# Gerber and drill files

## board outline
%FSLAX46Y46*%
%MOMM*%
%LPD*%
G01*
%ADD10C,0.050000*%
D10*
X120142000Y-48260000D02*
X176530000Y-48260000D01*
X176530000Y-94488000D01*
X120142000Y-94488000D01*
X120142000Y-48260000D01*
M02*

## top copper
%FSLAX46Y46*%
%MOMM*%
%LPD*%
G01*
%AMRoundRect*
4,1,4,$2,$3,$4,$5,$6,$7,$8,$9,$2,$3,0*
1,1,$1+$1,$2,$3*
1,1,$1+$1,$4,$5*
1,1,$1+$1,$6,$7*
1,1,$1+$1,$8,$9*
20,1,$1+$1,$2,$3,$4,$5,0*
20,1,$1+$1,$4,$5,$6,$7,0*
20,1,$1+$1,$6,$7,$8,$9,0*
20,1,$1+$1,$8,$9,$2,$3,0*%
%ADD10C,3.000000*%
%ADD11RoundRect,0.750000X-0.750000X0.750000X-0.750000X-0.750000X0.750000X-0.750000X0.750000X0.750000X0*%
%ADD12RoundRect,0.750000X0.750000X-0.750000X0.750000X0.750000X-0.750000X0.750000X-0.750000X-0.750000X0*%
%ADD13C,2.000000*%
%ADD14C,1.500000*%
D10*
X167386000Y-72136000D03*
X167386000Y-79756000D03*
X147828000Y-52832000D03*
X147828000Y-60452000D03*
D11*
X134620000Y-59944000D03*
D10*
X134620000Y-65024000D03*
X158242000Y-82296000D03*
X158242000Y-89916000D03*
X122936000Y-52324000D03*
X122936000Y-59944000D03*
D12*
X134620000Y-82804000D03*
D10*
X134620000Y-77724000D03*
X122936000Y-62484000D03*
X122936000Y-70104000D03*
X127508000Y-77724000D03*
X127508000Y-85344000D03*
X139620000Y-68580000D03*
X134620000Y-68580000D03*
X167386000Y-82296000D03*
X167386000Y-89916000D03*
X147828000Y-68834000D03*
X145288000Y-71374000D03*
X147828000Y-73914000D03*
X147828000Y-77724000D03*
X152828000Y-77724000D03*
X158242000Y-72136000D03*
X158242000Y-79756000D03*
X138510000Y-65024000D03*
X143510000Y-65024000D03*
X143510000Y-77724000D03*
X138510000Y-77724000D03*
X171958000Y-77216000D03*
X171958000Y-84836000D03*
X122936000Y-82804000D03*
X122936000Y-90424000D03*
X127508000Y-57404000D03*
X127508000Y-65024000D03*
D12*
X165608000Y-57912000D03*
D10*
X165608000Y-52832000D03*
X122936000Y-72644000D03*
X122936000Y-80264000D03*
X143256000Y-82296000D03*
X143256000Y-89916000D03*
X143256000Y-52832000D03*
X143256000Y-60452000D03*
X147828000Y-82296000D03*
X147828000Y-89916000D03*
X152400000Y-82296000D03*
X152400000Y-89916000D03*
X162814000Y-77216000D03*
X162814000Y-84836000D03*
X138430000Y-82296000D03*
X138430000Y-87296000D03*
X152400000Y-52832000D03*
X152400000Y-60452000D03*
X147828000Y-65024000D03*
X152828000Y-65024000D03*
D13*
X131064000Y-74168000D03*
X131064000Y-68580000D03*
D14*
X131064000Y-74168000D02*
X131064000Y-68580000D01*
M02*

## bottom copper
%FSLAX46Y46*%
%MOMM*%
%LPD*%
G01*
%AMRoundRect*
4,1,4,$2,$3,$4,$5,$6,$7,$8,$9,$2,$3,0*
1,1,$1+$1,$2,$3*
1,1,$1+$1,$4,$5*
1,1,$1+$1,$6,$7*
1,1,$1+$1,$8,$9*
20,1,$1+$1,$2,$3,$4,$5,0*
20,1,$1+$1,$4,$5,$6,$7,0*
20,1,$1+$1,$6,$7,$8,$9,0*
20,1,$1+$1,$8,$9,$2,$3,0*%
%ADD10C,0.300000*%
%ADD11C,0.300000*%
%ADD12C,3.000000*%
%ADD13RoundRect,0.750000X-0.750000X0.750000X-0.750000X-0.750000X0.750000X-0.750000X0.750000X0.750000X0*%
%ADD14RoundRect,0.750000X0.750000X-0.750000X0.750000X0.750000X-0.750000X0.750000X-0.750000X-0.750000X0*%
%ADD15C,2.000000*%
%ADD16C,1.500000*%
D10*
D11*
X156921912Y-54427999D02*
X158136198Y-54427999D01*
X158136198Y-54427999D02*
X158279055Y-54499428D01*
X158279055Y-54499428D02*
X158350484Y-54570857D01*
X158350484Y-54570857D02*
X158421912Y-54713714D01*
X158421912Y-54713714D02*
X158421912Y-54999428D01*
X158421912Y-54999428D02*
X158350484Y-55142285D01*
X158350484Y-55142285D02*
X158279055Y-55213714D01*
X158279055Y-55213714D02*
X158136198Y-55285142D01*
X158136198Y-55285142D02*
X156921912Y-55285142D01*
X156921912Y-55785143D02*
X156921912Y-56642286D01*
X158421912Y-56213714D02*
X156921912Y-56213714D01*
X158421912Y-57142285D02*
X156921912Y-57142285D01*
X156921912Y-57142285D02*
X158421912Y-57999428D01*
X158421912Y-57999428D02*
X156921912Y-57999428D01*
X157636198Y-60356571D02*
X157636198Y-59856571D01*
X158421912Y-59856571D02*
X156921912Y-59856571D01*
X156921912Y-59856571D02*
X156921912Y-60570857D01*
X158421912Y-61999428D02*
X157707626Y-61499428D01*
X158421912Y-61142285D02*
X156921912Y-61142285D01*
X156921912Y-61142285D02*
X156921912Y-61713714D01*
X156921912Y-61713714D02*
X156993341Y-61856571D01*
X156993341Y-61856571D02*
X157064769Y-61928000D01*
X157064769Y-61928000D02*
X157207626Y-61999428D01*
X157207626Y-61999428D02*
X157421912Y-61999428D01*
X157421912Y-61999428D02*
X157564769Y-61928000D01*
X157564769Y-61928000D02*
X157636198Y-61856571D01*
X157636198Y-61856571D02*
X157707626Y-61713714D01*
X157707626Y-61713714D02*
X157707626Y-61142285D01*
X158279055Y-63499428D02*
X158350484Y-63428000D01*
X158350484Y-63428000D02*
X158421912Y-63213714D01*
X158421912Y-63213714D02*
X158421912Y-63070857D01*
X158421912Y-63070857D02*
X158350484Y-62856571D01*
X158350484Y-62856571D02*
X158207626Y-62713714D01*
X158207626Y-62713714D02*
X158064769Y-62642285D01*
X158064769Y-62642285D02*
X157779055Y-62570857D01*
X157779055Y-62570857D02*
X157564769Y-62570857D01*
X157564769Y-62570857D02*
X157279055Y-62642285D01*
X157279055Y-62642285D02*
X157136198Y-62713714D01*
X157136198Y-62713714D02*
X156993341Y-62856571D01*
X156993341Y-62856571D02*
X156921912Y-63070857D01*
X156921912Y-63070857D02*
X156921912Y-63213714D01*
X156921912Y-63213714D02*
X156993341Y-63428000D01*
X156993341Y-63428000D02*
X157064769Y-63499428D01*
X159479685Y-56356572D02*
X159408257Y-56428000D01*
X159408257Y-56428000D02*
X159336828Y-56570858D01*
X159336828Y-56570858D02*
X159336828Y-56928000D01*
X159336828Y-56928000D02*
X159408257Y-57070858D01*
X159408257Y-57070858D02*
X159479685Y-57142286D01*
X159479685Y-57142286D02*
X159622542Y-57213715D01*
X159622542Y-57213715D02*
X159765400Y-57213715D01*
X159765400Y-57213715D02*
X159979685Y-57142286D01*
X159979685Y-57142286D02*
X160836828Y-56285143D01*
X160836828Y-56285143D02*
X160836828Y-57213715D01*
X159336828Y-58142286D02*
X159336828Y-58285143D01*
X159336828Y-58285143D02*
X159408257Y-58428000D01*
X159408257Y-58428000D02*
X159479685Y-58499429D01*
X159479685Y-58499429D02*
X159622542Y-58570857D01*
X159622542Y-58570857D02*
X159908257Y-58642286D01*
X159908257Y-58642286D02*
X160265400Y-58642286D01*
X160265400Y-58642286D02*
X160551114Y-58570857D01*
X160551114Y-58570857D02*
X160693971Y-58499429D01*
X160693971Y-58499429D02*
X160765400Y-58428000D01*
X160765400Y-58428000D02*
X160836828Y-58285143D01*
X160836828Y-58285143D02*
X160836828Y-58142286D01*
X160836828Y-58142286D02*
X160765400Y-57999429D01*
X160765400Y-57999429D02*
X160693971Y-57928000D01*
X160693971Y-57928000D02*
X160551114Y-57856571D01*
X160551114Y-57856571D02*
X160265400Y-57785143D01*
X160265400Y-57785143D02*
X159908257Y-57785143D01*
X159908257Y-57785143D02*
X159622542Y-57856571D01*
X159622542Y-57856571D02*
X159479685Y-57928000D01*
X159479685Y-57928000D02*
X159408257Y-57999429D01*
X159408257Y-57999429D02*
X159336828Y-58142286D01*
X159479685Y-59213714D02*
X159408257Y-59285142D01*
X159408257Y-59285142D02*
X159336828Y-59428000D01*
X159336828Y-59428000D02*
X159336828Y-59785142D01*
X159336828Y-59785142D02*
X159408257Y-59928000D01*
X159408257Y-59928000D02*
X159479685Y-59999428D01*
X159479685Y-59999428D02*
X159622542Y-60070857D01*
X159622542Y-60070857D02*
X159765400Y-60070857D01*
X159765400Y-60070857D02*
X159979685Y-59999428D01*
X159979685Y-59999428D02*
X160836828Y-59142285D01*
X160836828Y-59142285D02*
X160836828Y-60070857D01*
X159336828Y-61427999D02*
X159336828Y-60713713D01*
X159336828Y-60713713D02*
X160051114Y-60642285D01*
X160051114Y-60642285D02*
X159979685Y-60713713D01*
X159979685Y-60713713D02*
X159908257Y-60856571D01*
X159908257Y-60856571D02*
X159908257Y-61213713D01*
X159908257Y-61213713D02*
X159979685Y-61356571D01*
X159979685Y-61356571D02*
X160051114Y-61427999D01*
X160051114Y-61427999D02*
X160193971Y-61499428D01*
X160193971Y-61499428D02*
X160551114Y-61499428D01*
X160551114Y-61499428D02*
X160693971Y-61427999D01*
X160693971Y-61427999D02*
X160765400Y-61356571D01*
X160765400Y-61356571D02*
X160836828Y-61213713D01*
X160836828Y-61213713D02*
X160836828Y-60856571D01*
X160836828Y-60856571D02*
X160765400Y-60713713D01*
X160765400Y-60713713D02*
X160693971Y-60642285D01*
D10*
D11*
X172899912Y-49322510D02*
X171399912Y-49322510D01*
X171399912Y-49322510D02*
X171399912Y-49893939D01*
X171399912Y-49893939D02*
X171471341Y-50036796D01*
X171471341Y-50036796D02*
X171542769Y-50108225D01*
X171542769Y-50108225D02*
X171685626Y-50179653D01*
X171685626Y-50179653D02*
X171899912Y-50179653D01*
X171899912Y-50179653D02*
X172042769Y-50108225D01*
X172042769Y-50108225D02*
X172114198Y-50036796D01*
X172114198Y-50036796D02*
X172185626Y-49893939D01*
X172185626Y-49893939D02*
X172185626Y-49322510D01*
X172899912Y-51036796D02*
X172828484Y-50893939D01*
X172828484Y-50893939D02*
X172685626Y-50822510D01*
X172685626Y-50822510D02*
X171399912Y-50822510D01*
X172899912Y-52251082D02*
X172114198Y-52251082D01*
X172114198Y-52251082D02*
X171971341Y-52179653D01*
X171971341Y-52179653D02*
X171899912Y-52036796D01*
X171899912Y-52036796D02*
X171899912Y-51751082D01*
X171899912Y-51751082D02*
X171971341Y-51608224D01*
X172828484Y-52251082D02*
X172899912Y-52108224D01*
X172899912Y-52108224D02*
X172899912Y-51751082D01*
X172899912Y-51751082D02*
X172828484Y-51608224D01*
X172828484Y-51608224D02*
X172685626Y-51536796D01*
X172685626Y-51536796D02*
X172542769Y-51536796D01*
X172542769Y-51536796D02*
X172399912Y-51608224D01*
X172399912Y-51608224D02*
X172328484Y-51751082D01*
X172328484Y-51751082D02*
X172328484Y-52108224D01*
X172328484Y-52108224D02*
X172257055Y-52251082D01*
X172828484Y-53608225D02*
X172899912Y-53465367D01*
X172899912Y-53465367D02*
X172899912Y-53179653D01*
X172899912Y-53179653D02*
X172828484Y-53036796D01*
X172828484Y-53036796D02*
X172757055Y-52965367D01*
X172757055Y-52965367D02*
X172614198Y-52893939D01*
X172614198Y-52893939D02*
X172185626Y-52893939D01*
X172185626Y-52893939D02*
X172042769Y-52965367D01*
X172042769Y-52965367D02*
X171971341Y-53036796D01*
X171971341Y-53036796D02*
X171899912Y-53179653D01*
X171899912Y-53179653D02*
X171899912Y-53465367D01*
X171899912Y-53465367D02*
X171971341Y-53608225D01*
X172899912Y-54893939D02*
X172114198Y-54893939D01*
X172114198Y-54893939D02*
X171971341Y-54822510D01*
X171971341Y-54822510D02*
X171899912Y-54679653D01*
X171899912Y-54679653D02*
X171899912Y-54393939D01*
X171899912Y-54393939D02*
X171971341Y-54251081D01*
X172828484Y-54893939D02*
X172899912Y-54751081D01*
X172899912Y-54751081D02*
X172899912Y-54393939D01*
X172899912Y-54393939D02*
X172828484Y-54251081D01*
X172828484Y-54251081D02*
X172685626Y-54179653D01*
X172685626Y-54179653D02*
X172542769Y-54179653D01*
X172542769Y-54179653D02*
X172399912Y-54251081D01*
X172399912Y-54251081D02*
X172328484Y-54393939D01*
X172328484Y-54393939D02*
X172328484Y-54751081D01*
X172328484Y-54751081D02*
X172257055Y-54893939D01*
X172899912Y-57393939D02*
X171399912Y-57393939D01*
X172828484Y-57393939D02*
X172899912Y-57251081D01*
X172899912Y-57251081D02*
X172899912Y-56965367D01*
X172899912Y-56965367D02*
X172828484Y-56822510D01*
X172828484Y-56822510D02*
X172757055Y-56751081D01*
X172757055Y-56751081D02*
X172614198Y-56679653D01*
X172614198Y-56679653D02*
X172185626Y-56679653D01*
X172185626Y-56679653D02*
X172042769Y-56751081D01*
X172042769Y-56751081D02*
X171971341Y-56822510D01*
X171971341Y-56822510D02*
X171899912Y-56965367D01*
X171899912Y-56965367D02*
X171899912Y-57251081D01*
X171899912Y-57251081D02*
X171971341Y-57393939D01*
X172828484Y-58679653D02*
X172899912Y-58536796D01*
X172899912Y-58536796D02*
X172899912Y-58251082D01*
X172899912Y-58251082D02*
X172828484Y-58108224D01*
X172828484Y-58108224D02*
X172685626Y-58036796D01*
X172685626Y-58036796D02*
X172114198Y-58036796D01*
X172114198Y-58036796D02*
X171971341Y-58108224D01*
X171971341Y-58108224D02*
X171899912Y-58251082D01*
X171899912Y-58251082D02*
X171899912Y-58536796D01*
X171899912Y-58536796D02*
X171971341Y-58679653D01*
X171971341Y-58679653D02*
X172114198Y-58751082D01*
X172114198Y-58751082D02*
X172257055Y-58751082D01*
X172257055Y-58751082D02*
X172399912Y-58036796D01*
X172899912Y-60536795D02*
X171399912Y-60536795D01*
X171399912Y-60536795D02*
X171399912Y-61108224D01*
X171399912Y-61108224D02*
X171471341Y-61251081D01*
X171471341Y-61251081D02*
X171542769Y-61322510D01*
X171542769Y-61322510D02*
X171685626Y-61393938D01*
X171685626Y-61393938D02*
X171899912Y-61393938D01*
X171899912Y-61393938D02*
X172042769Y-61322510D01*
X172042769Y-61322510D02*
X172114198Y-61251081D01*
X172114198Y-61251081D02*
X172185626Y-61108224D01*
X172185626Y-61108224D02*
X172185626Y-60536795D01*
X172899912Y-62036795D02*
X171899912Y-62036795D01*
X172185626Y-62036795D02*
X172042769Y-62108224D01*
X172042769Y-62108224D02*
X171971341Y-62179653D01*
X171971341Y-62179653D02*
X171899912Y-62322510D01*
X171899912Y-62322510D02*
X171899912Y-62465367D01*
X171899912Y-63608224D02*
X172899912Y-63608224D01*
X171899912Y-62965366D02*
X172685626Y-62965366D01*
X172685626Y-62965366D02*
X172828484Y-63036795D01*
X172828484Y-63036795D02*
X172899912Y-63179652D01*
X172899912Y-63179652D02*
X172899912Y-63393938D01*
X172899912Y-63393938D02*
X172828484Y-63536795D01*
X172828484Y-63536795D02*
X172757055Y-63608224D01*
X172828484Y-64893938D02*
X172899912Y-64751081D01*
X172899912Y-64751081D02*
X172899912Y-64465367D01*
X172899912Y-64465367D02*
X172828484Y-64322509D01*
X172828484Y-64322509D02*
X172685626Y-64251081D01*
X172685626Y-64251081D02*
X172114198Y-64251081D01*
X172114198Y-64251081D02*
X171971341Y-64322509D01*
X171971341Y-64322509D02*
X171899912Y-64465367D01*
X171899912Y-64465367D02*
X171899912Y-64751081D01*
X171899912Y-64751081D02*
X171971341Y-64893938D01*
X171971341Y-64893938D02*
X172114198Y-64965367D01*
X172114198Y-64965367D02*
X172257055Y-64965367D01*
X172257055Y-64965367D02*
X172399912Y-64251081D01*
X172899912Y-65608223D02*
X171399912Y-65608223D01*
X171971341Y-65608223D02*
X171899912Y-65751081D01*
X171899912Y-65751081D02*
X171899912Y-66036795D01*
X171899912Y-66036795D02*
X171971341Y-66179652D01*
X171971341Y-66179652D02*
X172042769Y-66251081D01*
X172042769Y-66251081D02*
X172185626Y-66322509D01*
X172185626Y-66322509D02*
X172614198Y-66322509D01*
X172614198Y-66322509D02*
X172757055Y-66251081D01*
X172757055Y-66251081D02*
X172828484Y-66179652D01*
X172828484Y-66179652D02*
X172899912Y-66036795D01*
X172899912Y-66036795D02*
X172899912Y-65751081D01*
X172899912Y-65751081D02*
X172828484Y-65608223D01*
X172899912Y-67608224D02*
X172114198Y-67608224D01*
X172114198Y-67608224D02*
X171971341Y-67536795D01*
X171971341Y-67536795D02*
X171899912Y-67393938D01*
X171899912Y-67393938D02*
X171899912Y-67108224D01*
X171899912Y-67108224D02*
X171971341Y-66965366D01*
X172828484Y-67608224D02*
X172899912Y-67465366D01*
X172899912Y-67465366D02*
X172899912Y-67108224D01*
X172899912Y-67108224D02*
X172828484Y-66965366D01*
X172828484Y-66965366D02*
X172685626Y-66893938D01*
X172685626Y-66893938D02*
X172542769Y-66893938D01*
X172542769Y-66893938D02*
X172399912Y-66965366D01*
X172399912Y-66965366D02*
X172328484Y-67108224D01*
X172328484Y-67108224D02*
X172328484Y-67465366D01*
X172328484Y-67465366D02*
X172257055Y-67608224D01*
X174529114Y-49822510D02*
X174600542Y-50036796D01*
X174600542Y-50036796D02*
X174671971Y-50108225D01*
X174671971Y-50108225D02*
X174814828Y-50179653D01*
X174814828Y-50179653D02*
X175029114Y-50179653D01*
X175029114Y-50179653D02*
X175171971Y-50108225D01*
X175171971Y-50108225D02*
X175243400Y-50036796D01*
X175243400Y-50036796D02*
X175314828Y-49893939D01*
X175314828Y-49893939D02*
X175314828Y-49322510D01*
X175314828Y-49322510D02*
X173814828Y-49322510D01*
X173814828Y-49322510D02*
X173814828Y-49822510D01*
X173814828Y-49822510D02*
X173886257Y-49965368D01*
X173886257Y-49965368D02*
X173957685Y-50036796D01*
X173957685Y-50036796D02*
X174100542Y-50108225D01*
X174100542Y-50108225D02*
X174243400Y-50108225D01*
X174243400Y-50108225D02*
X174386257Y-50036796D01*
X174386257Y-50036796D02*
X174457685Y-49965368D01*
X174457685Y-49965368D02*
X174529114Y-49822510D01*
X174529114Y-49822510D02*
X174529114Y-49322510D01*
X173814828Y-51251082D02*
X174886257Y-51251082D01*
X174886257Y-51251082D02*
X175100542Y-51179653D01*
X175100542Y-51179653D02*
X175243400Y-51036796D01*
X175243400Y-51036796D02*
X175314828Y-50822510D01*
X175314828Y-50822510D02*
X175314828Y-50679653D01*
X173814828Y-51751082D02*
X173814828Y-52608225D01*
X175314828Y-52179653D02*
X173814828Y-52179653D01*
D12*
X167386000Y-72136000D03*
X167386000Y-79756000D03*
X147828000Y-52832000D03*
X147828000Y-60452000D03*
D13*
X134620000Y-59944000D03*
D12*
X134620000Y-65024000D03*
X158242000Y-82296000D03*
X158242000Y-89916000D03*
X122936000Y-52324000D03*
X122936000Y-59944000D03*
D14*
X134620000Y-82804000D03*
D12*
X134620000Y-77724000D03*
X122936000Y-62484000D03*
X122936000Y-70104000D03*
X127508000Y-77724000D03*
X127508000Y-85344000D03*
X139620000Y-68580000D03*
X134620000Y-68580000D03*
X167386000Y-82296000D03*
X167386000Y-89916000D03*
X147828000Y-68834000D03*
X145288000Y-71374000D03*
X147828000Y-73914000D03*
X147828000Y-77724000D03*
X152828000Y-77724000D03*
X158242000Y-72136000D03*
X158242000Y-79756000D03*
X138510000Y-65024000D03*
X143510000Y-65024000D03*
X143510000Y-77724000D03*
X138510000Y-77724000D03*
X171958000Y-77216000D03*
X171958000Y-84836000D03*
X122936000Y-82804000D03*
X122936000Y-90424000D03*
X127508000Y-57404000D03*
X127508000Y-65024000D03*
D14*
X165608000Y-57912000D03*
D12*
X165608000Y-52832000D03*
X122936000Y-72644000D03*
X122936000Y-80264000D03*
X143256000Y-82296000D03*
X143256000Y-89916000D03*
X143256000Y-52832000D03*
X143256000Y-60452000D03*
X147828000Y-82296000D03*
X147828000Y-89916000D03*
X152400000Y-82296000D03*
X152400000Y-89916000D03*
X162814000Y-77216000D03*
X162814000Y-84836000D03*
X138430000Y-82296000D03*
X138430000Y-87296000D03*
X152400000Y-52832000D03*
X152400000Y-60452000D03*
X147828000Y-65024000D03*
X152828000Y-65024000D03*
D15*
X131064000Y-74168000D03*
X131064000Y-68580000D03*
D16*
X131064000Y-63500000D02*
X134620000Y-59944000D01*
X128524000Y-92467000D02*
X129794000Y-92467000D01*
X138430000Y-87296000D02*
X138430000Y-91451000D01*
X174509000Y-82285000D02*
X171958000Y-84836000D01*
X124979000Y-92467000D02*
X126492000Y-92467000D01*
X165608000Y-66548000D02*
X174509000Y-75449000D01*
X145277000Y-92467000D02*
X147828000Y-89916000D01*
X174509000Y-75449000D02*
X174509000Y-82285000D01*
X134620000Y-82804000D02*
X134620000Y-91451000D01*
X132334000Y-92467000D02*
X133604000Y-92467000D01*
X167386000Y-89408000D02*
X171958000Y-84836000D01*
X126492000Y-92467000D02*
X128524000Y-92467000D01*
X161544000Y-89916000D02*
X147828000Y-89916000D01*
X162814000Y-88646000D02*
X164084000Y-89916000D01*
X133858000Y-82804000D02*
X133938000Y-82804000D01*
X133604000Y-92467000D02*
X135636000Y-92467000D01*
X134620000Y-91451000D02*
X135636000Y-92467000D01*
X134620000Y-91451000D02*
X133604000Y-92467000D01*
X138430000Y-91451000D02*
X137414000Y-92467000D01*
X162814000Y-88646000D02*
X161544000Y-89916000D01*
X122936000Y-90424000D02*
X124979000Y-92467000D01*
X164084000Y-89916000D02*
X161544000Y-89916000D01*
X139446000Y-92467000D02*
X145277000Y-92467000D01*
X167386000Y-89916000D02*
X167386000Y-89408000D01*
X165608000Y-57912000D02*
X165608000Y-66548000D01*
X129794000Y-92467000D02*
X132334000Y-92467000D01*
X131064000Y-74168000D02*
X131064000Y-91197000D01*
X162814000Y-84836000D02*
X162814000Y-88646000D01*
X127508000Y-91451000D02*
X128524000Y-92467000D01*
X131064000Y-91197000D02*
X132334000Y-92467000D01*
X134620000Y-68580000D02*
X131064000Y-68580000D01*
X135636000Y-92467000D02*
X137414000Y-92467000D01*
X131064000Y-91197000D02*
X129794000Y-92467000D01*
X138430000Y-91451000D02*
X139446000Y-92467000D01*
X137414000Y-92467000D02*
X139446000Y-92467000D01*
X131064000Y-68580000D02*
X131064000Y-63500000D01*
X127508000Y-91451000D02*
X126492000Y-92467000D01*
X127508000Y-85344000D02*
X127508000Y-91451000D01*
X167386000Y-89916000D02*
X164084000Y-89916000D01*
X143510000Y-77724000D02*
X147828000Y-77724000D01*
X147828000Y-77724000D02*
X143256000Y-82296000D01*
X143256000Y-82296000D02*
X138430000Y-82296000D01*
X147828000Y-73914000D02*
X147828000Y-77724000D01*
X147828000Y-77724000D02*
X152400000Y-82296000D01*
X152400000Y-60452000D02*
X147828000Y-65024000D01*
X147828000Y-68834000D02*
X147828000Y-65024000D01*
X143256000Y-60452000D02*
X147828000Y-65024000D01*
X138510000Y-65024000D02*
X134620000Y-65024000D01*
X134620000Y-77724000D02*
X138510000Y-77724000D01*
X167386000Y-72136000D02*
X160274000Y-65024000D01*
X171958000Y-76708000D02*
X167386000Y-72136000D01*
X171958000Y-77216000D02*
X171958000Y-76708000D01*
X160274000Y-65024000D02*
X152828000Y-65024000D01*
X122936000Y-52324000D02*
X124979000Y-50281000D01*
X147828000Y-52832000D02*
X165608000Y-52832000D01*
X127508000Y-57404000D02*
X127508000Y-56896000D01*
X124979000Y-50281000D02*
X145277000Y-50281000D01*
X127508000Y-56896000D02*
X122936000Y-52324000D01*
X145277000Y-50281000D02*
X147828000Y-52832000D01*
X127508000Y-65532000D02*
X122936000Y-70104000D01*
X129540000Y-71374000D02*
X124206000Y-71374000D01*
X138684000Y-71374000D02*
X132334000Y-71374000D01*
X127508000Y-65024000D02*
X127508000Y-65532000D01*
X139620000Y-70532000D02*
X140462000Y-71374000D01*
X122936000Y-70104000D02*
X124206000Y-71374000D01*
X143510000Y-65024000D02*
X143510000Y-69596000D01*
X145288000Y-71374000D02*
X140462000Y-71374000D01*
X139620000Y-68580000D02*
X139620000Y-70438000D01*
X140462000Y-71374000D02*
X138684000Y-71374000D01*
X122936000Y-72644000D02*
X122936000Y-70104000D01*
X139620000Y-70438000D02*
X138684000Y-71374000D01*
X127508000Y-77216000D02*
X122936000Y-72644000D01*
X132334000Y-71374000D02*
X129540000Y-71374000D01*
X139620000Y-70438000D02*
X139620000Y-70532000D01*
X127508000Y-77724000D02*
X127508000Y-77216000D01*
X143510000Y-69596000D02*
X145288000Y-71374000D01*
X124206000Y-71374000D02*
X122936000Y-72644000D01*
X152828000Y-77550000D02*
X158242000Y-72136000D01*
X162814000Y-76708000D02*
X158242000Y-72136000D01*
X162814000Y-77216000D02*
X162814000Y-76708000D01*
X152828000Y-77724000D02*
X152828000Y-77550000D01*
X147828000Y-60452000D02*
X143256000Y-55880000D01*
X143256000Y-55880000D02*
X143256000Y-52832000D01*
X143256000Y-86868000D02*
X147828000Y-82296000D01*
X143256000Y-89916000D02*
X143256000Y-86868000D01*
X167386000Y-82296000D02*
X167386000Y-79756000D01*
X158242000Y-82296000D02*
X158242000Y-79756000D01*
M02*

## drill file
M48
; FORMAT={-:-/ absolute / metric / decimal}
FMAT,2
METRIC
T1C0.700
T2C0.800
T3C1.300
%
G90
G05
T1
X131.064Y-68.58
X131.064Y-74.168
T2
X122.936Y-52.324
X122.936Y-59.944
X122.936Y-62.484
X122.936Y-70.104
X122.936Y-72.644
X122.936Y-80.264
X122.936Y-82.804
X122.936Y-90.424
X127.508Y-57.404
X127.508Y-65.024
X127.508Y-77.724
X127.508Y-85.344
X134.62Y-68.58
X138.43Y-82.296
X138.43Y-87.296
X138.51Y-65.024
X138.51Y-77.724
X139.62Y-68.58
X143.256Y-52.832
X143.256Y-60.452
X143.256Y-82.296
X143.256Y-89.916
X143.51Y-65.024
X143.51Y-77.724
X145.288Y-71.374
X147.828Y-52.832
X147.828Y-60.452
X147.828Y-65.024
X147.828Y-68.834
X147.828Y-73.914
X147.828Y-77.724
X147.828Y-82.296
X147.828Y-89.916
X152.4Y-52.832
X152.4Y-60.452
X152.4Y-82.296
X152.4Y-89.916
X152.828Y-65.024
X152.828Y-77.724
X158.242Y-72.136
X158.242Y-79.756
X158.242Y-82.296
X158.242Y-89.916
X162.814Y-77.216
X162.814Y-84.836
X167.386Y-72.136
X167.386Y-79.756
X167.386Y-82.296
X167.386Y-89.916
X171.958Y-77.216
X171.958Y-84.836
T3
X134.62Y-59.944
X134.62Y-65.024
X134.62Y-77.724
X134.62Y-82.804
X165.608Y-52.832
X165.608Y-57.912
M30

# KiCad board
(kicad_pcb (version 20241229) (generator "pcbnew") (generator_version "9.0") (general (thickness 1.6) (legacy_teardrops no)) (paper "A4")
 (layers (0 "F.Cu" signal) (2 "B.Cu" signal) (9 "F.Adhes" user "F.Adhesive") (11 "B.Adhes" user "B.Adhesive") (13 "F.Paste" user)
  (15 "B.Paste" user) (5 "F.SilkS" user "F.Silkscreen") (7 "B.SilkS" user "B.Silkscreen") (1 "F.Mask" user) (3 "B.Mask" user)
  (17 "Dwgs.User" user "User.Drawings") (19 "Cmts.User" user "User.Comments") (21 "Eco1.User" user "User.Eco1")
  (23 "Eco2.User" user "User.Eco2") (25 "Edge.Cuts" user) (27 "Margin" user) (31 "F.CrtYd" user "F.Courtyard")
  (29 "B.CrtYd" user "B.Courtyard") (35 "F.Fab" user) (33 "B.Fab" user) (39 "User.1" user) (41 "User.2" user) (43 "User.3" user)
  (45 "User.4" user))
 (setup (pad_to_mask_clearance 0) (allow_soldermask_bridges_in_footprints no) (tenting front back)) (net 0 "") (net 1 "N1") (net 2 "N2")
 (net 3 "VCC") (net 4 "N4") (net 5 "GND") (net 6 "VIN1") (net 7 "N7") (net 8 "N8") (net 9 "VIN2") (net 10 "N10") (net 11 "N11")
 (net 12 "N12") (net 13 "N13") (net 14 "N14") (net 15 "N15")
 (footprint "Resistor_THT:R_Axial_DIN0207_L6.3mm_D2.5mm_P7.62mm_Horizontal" (layer "F.Cu") (at 167.386 72.136 -90)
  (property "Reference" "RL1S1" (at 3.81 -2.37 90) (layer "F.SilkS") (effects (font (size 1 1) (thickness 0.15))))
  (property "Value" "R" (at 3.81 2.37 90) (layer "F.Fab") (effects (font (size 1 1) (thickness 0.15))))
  (pad "1" thru_hole circle (at 0 0 270) (size 3 3) (drill 0.8) (layers "*.Cu" "*.Mask") (remove_unused_layers no) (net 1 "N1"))
  (pad "2" thru_hole circle (at 7.62 0 270) (size 3 3) (drill 0.8) (layers "*.Cu" "*.Mask") (remove_unused_layers no) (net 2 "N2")))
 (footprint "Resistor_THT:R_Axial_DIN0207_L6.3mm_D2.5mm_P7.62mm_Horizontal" (layer "F.Cu") (at 147.828 52.832 -90)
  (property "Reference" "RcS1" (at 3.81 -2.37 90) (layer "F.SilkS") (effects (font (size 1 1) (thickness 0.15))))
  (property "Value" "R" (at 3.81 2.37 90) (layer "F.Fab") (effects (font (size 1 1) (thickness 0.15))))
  (pad "1" thru_hole circle (at 0 0 270) (size 3 3) (drill 0.8) (layers "*.Cu" "*.Mask") (remove_unused_layers no) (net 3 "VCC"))
  (pad "2" thru_hole circle (at 7.62 0 270) (size 3 3) (drill 0.8) (layers "*.Cu" "*.Mask") (remove_unused_layers no) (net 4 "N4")))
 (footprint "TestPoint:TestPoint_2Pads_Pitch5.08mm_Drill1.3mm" (layer "F.Cu") (at 134.62 59.944 -90)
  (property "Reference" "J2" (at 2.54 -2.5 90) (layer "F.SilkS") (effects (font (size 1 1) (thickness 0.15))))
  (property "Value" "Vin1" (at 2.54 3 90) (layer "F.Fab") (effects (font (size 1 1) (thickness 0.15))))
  (pad "1" thru_hole roundrect (at 0 0 270) (size 3 3) (drill 1.3) (layers "*.Cu" "*.Mask") (remove_unused_layers no)
   (roundrect_rratio 0.25) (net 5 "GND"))
  (pad "2" thru_hole circle (at 5.08 0 270) (size 3 3) (drill 1.3) (layers "*.Cu" "*.Mask") (remove_unused_layers no) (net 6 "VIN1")))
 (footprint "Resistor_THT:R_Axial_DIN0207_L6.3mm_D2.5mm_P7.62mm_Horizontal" (layer "F.Cu") (at 158.242 82.296 -90)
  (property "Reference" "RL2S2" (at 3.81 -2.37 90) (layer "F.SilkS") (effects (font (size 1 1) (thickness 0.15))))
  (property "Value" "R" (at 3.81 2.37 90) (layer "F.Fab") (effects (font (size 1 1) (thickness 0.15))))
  (pad "1" thru_hole circle (at 0 0 270) (size 3 3) (drill 0.8) (layers "*.Cu" "*.Mask") (remove_unused_layers no) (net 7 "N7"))
  (pad "2" thru_hole circle (at 7.62 0 270) (size 3 3) (drill 0.8) (layers "*.Cu" "*.Mask") (remove_unused_layers no) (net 5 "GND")))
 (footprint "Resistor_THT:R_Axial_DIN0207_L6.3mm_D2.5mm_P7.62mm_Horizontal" (layer "F.Cu") (at 122.936 52.324 -90)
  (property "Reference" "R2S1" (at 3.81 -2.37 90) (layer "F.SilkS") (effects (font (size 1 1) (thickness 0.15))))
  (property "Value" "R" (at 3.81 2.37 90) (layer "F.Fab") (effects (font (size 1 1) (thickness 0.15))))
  (pad "1" thru_hole circle (at 0 0 270) (size 3 3) (drill 0.8) (layers "*.Cu" "*.Mask") (remove_unused_layers no) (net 3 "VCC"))
  (pad "2" thru_hole circle (at 7.62 0 270) (size 3 3) (drill 0.8) (layers "*.Cu" "*.Mask") (remove_unused_layers no) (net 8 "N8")))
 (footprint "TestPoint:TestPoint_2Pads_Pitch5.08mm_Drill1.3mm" (layer "F.Cu") (at 134.62 82.804 90)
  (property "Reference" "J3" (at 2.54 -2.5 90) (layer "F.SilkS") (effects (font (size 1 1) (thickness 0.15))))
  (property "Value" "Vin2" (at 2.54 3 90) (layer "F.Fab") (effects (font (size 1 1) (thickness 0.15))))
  (pad "1" thru_hole roundrect (at 0 0 90) (size 3 3) (drill 1.3) (layers "*.Cu" "*.Mask") (remove_unused_layers no) (roundrect_rratio 0.25)
   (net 5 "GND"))
  (pad "2" thru_hole circle (at 5.08 0 90) (size 3 3) (drill 1.3) (layers "*.Cu" "*.Mask") (remove_unused_layers no) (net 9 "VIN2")))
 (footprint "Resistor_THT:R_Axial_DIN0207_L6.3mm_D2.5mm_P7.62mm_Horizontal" (layer "F.Cu") (at 122.936 62.484 -90)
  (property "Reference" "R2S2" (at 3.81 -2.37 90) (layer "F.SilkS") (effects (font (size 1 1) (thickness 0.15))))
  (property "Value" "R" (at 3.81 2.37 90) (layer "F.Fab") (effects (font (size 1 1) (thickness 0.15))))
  (pad "1" thru_hole circle (at 0 0 270) (size 3 3) (drill 0.8) (layers "*.Cu" "*.Mask") (remove_unused_layers no) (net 8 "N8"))
  (pad "2" thru_hole circle (at 7.62 0 270) (size 3 3) (drill 0.8) (layers "*.Cu" "*.Mask") (remove_unused_layers no) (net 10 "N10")))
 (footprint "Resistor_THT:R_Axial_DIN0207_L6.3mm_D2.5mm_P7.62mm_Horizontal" (layer "F.Cu") (at 127.508 77.724 -90)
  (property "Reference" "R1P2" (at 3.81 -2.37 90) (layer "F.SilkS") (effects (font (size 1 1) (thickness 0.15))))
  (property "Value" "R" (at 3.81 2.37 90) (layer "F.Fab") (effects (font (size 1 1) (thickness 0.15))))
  (pad "1" thru_hole circle (at 0 0 270) (size 3 3) (drill 0.8) (layers "*.Cu" "*.Mask") (remove_unused_layers no) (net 10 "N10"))
  (pad "2" thru_hole circle (at 7.62 0 270) (size 3 3) (drill 0.8) (layers "*.Cu" "*.Mask") (remove_unused_layers no) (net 5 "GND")))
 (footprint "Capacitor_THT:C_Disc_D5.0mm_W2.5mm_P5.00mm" (layer "F.Cu") (at 139.62 68.58 180)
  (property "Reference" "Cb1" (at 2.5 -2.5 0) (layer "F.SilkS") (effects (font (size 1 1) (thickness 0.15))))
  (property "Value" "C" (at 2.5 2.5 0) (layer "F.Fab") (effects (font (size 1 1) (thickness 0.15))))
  (pad "1" thru_hole circle (at 0 0 180) (size 3 3) (drill 0.8) (layers "*.Cu" "*.Mask") (remove_unused_layers no) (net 10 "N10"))
  (pad "2" thru_hole circle (at 5 0 180) (size 3 3) (drill 0.8) (layers "*.Cu" "*.Mask") (remove_unused_layers no) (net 5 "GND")))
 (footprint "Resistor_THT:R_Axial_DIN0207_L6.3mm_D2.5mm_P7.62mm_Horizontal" (layer "F.Cu") (at 167.386 82.296 -90)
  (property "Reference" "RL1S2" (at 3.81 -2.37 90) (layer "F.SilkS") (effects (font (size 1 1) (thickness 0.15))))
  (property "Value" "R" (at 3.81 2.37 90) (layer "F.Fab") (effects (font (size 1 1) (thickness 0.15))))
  (pad "1" thru_hole circle (at 0 0 270) (size 3 3) (drill 0.8) (layers "*.Cu" "*.Mask") (remove_unused_layers no) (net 2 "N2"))
  (pad "2" thru_hole circle (at 7.62 0 270) (size 3 3) (drill 0.8) (layers "*.Cu" "*.Mask") (remove_unused_layers no) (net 5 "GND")))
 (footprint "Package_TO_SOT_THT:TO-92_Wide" (layer "F.Cu") (at 147.828 73.914 90)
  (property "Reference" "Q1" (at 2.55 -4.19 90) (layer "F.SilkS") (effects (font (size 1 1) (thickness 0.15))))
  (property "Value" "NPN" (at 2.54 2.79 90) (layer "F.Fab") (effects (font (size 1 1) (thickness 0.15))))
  (pad "1" thru_hole circle (at 5.08 0 90) (size 3 3) (drill 0.8) (layers "*.Cu" "*.Mask") (remove_unused_layers no) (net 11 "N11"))
  (pad "2" thru_hole circle (at 2.54 -2.54 90) (size 3 3) (drill 0.8) (layers "*.Cu" "*.Mask") (remove_unused_layers no) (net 10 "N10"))
  (pad "3" thru_hole circle (at 0 0 90) (size 3 3) (drill 0.8) (layers "*.Cu" "*.Mask") (remove_unused_layers no) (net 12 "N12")))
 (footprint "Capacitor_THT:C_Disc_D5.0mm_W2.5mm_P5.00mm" (layer "F.Cu") (at 147.828 77.724)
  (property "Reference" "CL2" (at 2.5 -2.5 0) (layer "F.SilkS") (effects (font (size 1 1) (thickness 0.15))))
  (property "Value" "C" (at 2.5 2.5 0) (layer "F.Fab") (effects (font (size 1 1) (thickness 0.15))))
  (pad "1" thru_hole circle (at 0 0) (size 3 3) (drill 0.8) (layers "*.Cu" "*.Mask") (remove_unused_layers no) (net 12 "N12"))
  (pad "2" thru_hole circle (at 5 0) (size 3 3) (drill 0.8) (layers "*.Cu" "*.Mask") (remove_unused_layers no) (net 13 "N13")))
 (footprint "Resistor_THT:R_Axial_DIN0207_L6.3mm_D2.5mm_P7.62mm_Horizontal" (layer "F.Cu") (at 158.242 72.136 -90)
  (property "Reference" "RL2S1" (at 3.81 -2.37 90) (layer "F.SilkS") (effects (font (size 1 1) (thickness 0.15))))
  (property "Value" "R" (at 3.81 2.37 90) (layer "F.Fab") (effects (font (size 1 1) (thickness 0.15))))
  (pad "1" thru_hole circle (at 0 0 270) (size 3 3) (drill 0.8) (layers "*.Cu" "*.Mask") (remove_unused_layers no) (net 13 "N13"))
  (pad "2" thru_hole circle (at 7.62 0 270) (size 3 3) (drill 0.8) (layers "*.Cu" "*.Mask") (remove_unused_layers no) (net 7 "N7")))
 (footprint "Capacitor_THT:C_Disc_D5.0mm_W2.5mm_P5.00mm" (layer "F.Cu") (at 138.51 65.024)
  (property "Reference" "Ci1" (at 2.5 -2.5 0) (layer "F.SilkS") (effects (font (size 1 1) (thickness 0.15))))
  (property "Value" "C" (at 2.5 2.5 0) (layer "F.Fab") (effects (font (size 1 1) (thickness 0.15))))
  (pad "1" thru_hole circle (at 0 0) (size 3 3) (drill 0.8) (layers "*.Cu" "*.Mask") (remove_unused_layers no) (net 6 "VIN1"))
  (pad "2" thru_hole circle (at 5 0) (size 3 3) (drill 0.8) (layers "*.Cu" "*.Mask") (remove_unused_layers no) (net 10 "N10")))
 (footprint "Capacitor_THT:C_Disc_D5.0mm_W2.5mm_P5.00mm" (layer "F.Cu") (at 143.51 77.724 180)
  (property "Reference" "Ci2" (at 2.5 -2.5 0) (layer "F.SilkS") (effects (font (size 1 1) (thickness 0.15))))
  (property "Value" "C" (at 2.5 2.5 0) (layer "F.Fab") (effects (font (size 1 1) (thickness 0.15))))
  (pad "1" thru_hole circle (at 0 0 180) (size 3 3) (drill 0.8) (layers "*.Cu" "*.Mask") (remove_unused_layers no) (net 12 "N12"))
  (pad "2" thru_hole circle (at 5 0 180) (size 3 3) (drill 0.8) (layers "*.Cu" "*.Mask") (remove_unused_layers no) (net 9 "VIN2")))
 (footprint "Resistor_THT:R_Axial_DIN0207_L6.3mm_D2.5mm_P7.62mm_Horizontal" (layer "F.Cu") (at 171.958 77.216 -90)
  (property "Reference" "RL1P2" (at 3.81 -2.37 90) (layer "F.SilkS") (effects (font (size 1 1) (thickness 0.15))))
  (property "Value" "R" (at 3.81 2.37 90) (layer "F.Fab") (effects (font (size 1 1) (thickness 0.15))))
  (pad "1" thru_hole circle (at 0 0 270) (size 3 3) (drill 0.8) (layers "*.Cu" "*.Mask") (remove_unused_layers no) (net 1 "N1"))
  (pad "2" thru_hole circle (at 7.62 0 270) (size 3 3) (drill 0.8) (layers "*.Cu" "*.Mask") (remove_unused_layers no) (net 5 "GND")))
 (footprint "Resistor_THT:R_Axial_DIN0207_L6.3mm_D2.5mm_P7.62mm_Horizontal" (layer "F.Cu") (at 122.936 82.804 -90)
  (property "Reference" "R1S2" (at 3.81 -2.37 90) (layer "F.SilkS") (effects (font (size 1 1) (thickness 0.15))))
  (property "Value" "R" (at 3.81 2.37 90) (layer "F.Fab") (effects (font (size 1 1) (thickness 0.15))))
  (pad "1" thru_hole circle (at 0 0 270) (size 3 3) (drill 0.8) (layers "*.Cu" "*.Mask") (remove_unused_layers no) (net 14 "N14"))
  (pad "2" thru_hole circle (at 7.62 0 270) (size 3 3) (drill 0.8) (layers "*.Cu" "*.Mask") (remove_unused_layers no) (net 5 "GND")))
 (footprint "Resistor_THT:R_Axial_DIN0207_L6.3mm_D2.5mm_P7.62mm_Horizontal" (layer "F.Cu") (at 127.508 57.404 -90)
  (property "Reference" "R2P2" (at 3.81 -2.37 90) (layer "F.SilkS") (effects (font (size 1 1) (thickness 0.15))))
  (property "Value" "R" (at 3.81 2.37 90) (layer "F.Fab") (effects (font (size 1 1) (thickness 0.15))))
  (pad "1" thru_hole circle (at 0 0 270) (size 3 3) (drill 0.8) (layers "*.Cu" "*.Mask") (remove_unused_layers no) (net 3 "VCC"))
  (pad "2" thru_hole circle (at 7.62 0 270) (size 3 3) (drill 0.8) (layers "*.Cu" "*.Mask") (remove_unused_layers no) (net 10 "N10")))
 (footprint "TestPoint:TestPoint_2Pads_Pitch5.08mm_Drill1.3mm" (layer "F.Cu") (at 165.608 57.912 90)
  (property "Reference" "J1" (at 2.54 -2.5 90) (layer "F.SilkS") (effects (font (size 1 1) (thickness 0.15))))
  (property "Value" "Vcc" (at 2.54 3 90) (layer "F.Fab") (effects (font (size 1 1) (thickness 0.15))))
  (pad "1" thru_hole roundrect (at 0 0 90) (size 3 3) (drill 1.3) (layers "*.Cu" "*.Mask") (remove_unused_layers no) (roundrect_rratio 0.25)
   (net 5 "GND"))
  (pad "2" thru_hole circle (at 5.08 0 90) (size 3 3) (drill 1.3) (layers "*.Cu" "*.Mask") (remove_unused_layers no) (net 3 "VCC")))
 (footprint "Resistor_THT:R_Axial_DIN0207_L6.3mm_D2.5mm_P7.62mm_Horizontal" (layer "F.Cu") (at 122.936 72.644 -90)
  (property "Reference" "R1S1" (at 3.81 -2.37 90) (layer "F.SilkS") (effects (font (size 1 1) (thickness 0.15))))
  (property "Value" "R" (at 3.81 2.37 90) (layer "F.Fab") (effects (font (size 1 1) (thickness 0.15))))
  (pad "1" thru_hole circle (at 0 0 270) (size 3 3) (drill 0.8) (layers "*.Cu" "*.Mask") (remove_unused_layers no) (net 10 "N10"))
  (pad "2" thru_hole circle (at 7.62 0 270) (size 3 3) (drill 0.8) (layers "*.Cu" "*.Mask") (remove_unused_layers no) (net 14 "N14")))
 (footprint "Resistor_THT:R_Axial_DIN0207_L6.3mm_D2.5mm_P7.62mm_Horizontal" (layer "F.Cu") (at 143.256 82.296 -90)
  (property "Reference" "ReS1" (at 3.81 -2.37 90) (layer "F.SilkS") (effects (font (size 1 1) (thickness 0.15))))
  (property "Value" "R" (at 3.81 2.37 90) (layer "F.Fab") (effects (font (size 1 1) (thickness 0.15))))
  (pad "1" thru_hole circle (at 0 0 270) (size 3 3) (drill 0.8) (layers "*.Cu" "*.Mask") (remove_unused_layers no) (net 12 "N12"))
  (pad "2" thru_hole circle (at 7.62 0 270) (size 3 3) (drill 0.8) (layers "*.Cu" "*.Mask") (remove_unused_layers no) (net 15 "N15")))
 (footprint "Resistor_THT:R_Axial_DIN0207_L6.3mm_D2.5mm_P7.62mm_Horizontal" (layer "F.Cu") (at 143.256 52.832 -90)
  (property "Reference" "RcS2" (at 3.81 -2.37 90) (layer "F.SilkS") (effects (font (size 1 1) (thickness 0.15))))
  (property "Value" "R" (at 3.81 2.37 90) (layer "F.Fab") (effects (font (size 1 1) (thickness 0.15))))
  (pad "1" thru_hole circle (at 0 0 270) (size 3 3) (drill 0.8) (layers "*.Cu" "*.Mask") (remove_unused_layers no) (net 4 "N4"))
  (pad "2" thru_hole circle (at 7.62 0 270) (size 3 3) (drill 0.8) (layers "*.Cu" "*.Mask") (remove_unused_layers no) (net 11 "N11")))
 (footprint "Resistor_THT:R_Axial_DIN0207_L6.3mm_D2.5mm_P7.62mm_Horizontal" (layer "F.Cu") (at 147.828 82.296 -90)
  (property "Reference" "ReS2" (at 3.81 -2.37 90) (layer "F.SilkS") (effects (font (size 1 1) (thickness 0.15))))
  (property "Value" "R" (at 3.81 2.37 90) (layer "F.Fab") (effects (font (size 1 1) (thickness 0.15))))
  (pad "1" thru_hole circle (at 0 0 270) (size 3 3) (drill 0.8) (layers "*.Cu" "*.Mask") (remove_unused_layers no) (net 15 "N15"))
  (pad "2" thru_hole circle (at 7.62 0 270) (size 3 3) (drill 0.8) (layers "*.Cu" "*.Mask") (remove_unused_layers no) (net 5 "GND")))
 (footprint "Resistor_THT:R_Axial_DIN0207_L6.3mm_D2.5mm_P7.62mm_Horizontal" (layer "F.Cu") (at 152.4 82.296 -90)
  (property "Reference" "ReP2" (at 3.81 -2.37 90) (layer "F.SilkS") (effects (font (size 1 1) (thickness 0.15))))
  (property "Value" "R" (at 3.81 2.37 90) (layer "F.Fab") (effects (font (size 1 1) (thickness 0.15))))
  (pad "1" thru_hole circle (at 0 0 270) (size 3 3) (drill 0.8) (layers "*.Cu" "*.Mask") (remove_unused_layers no) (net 12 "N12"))
  (pad "2" thru_hole circle (at 7.62 0 270) (size 3 3) (drill 0.8) (layers "*.Cu" "*.Mask") (remove_unused_layers no) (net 5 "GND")))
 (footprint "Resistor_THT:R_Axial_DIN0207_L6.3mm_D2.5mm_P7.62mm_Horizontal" (layer "F.Cu") (at 162.814 77.216 -90)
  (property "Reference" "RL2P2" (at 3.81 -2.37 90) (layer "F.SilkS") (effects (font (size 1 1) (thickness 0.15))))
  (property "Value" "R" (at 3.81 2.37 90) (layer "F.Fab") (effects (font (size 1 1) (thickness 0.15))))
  (pad "1" thru_hole circle (at 0 0 270) (size 3 3) (drill 0.8) (layers "*.Cu" "*.Mask") (remove_unused_layers no) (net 13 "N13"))
  (pad "2" thru_hole circle (at 7.62 0 270) (size 3 3) (drill 0.8) (layers "*.Cu" "*.Mask") (remove_unused_layers no) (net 5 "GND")))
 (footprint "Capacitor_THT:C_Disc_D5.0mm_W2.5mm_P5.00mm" (layer "F.Cu") (at 138.43 82.296 -90)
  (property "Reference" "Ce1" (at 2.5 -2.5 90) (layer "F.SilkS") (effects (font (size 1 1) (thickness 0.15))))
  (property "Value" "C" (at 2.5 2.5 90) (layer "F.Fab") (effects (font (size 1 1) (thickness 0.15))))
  (pad "1" thru_hole circle (at 0 0 270) (size 3 3) (drill 0.8) (layers "*.Cu" "*.Mask") (remove_unused_layers no) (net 12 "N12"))
  (pad "2" thru_hole circle (at 5 0 270) (size 3 3) (drill 0.8) (layers "*.Cu" "*.Mask") (remove_unused_layers no) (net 5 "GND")))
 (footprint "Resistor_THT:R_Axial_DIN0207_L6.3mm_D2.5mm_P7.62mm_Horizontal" (layer "F.Cu") (at 152.4 52.832 -90)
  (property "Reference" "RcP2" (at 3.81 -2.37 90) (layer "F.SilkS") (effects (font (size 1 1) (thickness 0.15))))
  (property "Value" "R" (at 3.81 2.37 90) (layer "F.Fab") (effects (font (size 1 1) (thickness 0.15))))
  (pad "1" thru_hole circle (at 0 0 270) (size 3 3) (drill 0.8) (layers "*.Cu" "*.Mask") (remove_unused_layers no) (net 3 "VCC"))
  (pad "2" thru_hole circle (at 7.62 0 270) (size 3 3) (drill 0.8) (layers "*.Cu" "*.Mask") (remove_unused_layers no) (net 11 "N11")))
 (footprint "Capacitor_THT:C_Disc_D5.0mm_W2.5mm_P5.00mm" (layer "F.Cu") (at 147.828 65.024)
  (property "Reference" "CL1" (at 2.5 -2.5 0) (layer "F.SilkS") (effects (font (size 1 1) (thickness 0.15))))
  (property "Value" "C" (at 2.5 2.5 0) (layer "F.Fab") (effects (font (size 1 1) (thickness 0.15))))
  (pad "1" thru_hole circle (at 0 0) (size 3 3) (drill 0.8) (layers "*.Cu" "*.Mask") (remove_unused_layers no) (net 11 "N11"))
  (pad "2" thru_hole circle (at 5 0) (size 3 3) (drill 0.8) (layers "*.Cu" "*.Mask") (remove_unused_layers no) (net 1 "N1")))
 (gr_rect (start 120.142 48.26) (end 176.53 94.488) (stroke (width 0.05) (type default)) (fill no) (layer "Edge.Cuts"))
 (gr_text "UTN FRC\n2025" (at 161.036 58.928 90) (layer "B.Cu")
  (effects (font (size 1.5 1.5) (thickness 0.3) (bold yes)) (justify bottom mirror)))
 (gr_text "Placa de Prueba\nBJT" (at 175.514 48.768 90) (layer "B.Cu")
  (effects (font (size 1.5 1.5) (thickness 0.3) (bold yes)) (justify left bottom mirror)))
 (segment (start 131.064 74.168) (end 131.064 68.58) (width 1.5) (layer "F.Cu") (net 5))
 (via (at 131.064 74.168) (size 2) (drill 0.7) (layers "F.Cu" "B.Cu") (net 5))
 (via (at 131.064 68.58) (size 2) (drill 0.7) (layers "F.Cu" "B.Cu") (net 5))
 (segment (start 131.064 63.5) (end 134.62 59.944) (width 1.5) (layer "B.Cu") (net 5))
 (segment (start 128.524 92.467) (end 129.794 92.467) (width 1.5) (layer "B.Cu") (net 5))
 (segment (start 138.43 87.296) (end 138.43 91.451) (width 1.5) (layer "B.Cu") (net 5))
 (segment (start 174.509 82.285) (end 171.958 84.836) (width 1.5) (layer "B.Cu") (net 5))
 (segment (start 124.979 92.467) (end 126.492 92.467) (width 1.5) (layer "B.Cu") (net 5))
 (segment (start 165.608 66.548) (end 174.509 75.449) (width 1.5) (layer "B.Cu") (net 5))
 (segment (start 145.277 92.467) (end 147.828 89.916) (width 1.5) (layer "B.Cu") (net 5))
 (segment (start 174.509 75.449) (end 174.509 82.285) (width 1.5) (layer "B.Cu") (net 5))
 (segment (start 134.62 82.804) (end 134.62 91.451) (width 1.5) (layer "B.Cu") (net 5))
 (segment (start 132.334 92.467) (end 133.604 92.467) (width 1.5) (layer "B.Cu") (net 5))
 (segment (start 167.386 89.408) (end 171.958 84.836) (width 1.5) (layer "B.Cu") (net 5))
 (segment (start 126.492 92.467) (end 128.524 92.467) (width 1.5) (layer "B.Cu") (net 5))
 (segment (start 161.544 89.916) (end 147.828 89.916) (width 1.5) (layer "B.Cu") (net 5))
 (segment (start 162.814 88.646) (end 164.084 89.916) (width 1.5) (layer "B.Cu") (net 5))
 (segment (start 133.858 82.804) (end 133.938 82.804) (width 1.5) (layer "B.Cu") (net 5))
 (segment (start 133.604 92.467) (end 135.636 92.467) (width 1.5) (layer "B.Cu") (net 5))
 (segment (start 134.62 91.451) (end 135.636 92.467) (width 1.5) (layer "B.Cu") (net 5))
 (segment (start 134.62 91.451) (end 133.604 92.467) (width 1.5) (layer "B.Cu") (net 5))
 (segment (start 138.43 91.451) (end 137.414 92.467) (width 1.5) (layer "B.Cu") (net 5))
 (segment (start 162.814 88.646) (end 161.544 89.916) (width 1.5) (layer "B.Cu") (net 5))
 (segment (start 122.936 90.424) (end 124.979 92.467) (width 1.5) (layer "B.Cu") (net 5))
 (segment (start 164.084 89.916) (end 161.544 89.916) (width 1.5) (layer "B.Cu") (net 5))
 (segment (start 139.446 92.467) (end 145.277 92.467) (width 1.5) (layer "B.Cu") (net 5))
 (segment (start 167.386 89.916) (end 167.386 89.408) (width 1.5) (layer "B.Cu") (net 5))
 (segment (start 165.608 57.912) (end 165.608 66.548) (width 1.5) (layer "B.Cu") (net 5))
 (segment (start 129.794 92.467) (end 132.334 92.467) (width 1.5) (layer "B.Cu") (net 5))
 (segment (start 131.064 74.168) (end 131.064 91.197) (width 1.5) (layer "B.Cu") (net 5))
 (segment (start 162.814 84.836) (end 162.814 88.646) (width 1.5) (layer "B.Cu") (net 5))
 (segment (start 127.508 91.451) (end 128.524 92.467) (width 1.5) (layer "B.Cu") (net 5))
 (segment (start 131.064 91.197) (end 132.334 92.467) (width 1.5) (layer "B.Cu") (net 5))
 (segment (start 134.62 68.58) (end 131.064 68.58) (width 1.5) (layer "B.Cu") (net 5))
 (segment (start 135.636 92.467) (end 137.414 92.467) (width 1.5) (layer "B.Cu") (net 5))
 (segment (start 131.064 91.197) (end 129.794 92.467) (width 1.5) (layer "B.Cu") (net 5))
 (segment (start 138.43 91.451) (end 139.446 92.467) (width 1.5) (layer "B.Cu") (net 5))
 (segment (start 137.414 92.467) (end 139.446 92.467) (width 1.5) (layer "B.Cu") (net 5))
 (segment (start 131.064 68.58) (end 131.064 63.5) (width 1.5) (layer "B.Cu") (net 5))
 (segment (start 127.508 91.451) (end 126.492 92.467) (width 1.5) (layer "B.Cu") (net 5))
 (segment (start 127.508 85.344) (end 127.508 91.451) (width 1.5) (layer "B.Cu") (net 5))
 (segment (start 167.386 89.916) (end 164.084 89.916) (width 1.5) (layer "B.Cu") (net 5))
 (segment (start 143.51 77.724) (end 147.828 77.724) (width 1.5) (layer "B.Cu") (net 12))
 (segment (start 147.828 77.724) (end 143.256 82.296) (width 1.5) (layer "B.Cu") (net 12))
 (segment (start 143.256 82.296) (end 138.43 82.296) (width 1.5) (layer "B.Cu") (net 12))
 (segment (start 147.828 73.914) (end 147.828 77.724) (width 1.5) (layer "B.Cu") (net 12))
 (segment (start 147.828 77.724) (end 152.4 82.296) (width 1.5) (layer "B.Cu") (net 12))
 (segment (start 152.4 60.452) (end 147.828 65.024) (width 1.5) (layer "B.Cu") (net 11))
 (segment (start 147.828 68.834) (end 147.828 65.024) (width 1.5) (layer "B.Cu") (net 11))
 (segment (start 143.256 60.452) (end 147.828 65.024) (width 1.5) (layer "B.Cu") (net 11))
 (segment (start 138.51 65.024) (end 134.62 65.024) (width 1.5) (layer "B.Cu") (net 6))
 (segment (start 134.62 77.724) (end 138.51 77.724) (width 1.5) (layer "B.Cu") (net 9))
 (segment (start 167.386 72.136) (end 160.274 65.024) (width 1.5) (layer "B.Cu") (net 1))
 (segment (start 171.958 76.708) (end 167.386 72.136) (width 1.5) (layer "B.Cu") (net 1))
 (segment (start 171.958 77.216) (end 171.958 76.708) (width 1.5) (layer "B.Cu") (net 1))
 (segment (start 160.274 65.024) (end 152.828 65.024) (width 1.5) (layer "B.Cu") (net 1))
 (segment (start 122.936 52.324) (end 124.979 50.281) (width 1.5) (layer "B.Cu") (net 3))
 (segment (start 147.828 52.832) (end 165.608 52.832) (width 1.5) (layer "B.Cu") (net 3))
 (segment (start 127.508 57.404) (end 127.508 56.896) (width 1.5) (layer "B.Cu") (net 3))
 (segment (start 124.979 50.281) (end 145.277 50.281) (width 1.5) (layer "B.Cu") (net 3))
 (segment (start 127.508 56.896) (end 122.936 52.324) (width 1.5) (layer "B.Cu") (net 3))
 (segment (start 145.277 50.281) (end 147.828 52.832) (width 1.5) (layer "B.Cu") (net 3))
 (segment (start 127.508 65.532) (end 122.936 70.104) (width 1.5) (layer "B.Cu") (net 10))
 (segment (start 129.54 71.374) (end 124.206 71.374) (width 1.5) (layer "B.Cu") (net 10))
 (segment (start 138.684 71.374) (end 132.334 71.374) (width 1.5) (layer "B.Cu") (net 10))
 (segment (start 127.508 65.024) (end 127.508 65.532) (width 1.5) (layer "B.Cu") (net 10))
 (segment (start 139.62 70.532) (end 140.462 71.374) (width 1.5) (layer "B.Cu") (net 10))
 (segment (start 122.936 70.104) (end 124.206 71.374) (width 1.5) (layer "B.Cu") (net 10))
 (segment (start 143.51 65.024) (end 143.51 69.596) (width 1.5) (layer "B.Cu") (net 10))
 (segment (start 145.288 71.374) (end 140.462 71.374) (width 1.5) (layer "B.Cu") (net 10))
 (segment (start 139.62 68.58) (end 139.62 70.438) (width 1.5) (layer "B.Cu") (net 10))
 (segment (start 140.462 71.374) (end 138.684 71.374) (width 1.5) (layer "B.Cu") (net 10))
 (segment (start 122.936 72.644) (end 122.936 70.104) (width 1.5) (layer "B.Cu") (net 10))
 (segment (start 139.62 70.438) (end 138.684 71.374) (width 1.5) (layer "B.Cu") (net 10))
 (segment (start 127.508 77.216) (end 122.936 72.644) (width 1.5) (layer "B.Cu") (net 10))
 (segment (start 132.334 71.374) (end 129.54 71.374) (width 1.5) (layer "B.Cu") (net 10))
 (segment (start 139.62 70.438) (end 139.62 70.532) (width 1.5) (layer "B.Cu") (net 10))
 (segment (start 127.508 77.724) (end 127.508 77.216) (width 1.5) (layer "B.Cu") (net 10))
 (segment (start 143.51 69.596) (end 145.288 71.374) (width 1.5) (layer "B.Cu") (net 10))
 (segment (start 124.206 71.374) (end 122.936 72.644) (width 1.5) (layer "B.Cu") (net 10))
 (segment (start 152.828 77.55) (end 158.242 72.136) (width 1.5) (layer "B.Cu") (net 13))
 (segment (start 162.814 76.708) (end 158.242 72.136) (width 1.5) (layer "B.Cu") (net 13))
 (segment (start 162.814 77.216) (end 162.814 76.708) (width 1.5) (layer "B.Cu") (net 13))
 (segment (start 152.828 77.724) (end 152.828 77.55) (width 1.5) (layer "B.Cu") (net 13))
 (segment (start 147.828 60.452) (end 143.256 55.88) (width 1.5) (layer "B.Cu") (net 4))
 (segment (start 143.256 55.88) (end 143.256 52.832) (width 1.5) (layer "B.Cu") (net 4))
 (segment (start 143.256 86.868) (end 147.828 82.296) (width 1.5) (layer "B.Cu") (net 15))
 (segment (start 143.256 89.916) (end 143.256 86.868) (width 1.5) (layer "B.Cu") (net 15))
 (segment (start 167.386 82.296) (end 167.386 79.756) (width 1.5) (layer "B.Cu") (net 2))
 (segment (start 158.242 82.296) (end 158.242 79.756) (width 1.5) (layer "B.Cu") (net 7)))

